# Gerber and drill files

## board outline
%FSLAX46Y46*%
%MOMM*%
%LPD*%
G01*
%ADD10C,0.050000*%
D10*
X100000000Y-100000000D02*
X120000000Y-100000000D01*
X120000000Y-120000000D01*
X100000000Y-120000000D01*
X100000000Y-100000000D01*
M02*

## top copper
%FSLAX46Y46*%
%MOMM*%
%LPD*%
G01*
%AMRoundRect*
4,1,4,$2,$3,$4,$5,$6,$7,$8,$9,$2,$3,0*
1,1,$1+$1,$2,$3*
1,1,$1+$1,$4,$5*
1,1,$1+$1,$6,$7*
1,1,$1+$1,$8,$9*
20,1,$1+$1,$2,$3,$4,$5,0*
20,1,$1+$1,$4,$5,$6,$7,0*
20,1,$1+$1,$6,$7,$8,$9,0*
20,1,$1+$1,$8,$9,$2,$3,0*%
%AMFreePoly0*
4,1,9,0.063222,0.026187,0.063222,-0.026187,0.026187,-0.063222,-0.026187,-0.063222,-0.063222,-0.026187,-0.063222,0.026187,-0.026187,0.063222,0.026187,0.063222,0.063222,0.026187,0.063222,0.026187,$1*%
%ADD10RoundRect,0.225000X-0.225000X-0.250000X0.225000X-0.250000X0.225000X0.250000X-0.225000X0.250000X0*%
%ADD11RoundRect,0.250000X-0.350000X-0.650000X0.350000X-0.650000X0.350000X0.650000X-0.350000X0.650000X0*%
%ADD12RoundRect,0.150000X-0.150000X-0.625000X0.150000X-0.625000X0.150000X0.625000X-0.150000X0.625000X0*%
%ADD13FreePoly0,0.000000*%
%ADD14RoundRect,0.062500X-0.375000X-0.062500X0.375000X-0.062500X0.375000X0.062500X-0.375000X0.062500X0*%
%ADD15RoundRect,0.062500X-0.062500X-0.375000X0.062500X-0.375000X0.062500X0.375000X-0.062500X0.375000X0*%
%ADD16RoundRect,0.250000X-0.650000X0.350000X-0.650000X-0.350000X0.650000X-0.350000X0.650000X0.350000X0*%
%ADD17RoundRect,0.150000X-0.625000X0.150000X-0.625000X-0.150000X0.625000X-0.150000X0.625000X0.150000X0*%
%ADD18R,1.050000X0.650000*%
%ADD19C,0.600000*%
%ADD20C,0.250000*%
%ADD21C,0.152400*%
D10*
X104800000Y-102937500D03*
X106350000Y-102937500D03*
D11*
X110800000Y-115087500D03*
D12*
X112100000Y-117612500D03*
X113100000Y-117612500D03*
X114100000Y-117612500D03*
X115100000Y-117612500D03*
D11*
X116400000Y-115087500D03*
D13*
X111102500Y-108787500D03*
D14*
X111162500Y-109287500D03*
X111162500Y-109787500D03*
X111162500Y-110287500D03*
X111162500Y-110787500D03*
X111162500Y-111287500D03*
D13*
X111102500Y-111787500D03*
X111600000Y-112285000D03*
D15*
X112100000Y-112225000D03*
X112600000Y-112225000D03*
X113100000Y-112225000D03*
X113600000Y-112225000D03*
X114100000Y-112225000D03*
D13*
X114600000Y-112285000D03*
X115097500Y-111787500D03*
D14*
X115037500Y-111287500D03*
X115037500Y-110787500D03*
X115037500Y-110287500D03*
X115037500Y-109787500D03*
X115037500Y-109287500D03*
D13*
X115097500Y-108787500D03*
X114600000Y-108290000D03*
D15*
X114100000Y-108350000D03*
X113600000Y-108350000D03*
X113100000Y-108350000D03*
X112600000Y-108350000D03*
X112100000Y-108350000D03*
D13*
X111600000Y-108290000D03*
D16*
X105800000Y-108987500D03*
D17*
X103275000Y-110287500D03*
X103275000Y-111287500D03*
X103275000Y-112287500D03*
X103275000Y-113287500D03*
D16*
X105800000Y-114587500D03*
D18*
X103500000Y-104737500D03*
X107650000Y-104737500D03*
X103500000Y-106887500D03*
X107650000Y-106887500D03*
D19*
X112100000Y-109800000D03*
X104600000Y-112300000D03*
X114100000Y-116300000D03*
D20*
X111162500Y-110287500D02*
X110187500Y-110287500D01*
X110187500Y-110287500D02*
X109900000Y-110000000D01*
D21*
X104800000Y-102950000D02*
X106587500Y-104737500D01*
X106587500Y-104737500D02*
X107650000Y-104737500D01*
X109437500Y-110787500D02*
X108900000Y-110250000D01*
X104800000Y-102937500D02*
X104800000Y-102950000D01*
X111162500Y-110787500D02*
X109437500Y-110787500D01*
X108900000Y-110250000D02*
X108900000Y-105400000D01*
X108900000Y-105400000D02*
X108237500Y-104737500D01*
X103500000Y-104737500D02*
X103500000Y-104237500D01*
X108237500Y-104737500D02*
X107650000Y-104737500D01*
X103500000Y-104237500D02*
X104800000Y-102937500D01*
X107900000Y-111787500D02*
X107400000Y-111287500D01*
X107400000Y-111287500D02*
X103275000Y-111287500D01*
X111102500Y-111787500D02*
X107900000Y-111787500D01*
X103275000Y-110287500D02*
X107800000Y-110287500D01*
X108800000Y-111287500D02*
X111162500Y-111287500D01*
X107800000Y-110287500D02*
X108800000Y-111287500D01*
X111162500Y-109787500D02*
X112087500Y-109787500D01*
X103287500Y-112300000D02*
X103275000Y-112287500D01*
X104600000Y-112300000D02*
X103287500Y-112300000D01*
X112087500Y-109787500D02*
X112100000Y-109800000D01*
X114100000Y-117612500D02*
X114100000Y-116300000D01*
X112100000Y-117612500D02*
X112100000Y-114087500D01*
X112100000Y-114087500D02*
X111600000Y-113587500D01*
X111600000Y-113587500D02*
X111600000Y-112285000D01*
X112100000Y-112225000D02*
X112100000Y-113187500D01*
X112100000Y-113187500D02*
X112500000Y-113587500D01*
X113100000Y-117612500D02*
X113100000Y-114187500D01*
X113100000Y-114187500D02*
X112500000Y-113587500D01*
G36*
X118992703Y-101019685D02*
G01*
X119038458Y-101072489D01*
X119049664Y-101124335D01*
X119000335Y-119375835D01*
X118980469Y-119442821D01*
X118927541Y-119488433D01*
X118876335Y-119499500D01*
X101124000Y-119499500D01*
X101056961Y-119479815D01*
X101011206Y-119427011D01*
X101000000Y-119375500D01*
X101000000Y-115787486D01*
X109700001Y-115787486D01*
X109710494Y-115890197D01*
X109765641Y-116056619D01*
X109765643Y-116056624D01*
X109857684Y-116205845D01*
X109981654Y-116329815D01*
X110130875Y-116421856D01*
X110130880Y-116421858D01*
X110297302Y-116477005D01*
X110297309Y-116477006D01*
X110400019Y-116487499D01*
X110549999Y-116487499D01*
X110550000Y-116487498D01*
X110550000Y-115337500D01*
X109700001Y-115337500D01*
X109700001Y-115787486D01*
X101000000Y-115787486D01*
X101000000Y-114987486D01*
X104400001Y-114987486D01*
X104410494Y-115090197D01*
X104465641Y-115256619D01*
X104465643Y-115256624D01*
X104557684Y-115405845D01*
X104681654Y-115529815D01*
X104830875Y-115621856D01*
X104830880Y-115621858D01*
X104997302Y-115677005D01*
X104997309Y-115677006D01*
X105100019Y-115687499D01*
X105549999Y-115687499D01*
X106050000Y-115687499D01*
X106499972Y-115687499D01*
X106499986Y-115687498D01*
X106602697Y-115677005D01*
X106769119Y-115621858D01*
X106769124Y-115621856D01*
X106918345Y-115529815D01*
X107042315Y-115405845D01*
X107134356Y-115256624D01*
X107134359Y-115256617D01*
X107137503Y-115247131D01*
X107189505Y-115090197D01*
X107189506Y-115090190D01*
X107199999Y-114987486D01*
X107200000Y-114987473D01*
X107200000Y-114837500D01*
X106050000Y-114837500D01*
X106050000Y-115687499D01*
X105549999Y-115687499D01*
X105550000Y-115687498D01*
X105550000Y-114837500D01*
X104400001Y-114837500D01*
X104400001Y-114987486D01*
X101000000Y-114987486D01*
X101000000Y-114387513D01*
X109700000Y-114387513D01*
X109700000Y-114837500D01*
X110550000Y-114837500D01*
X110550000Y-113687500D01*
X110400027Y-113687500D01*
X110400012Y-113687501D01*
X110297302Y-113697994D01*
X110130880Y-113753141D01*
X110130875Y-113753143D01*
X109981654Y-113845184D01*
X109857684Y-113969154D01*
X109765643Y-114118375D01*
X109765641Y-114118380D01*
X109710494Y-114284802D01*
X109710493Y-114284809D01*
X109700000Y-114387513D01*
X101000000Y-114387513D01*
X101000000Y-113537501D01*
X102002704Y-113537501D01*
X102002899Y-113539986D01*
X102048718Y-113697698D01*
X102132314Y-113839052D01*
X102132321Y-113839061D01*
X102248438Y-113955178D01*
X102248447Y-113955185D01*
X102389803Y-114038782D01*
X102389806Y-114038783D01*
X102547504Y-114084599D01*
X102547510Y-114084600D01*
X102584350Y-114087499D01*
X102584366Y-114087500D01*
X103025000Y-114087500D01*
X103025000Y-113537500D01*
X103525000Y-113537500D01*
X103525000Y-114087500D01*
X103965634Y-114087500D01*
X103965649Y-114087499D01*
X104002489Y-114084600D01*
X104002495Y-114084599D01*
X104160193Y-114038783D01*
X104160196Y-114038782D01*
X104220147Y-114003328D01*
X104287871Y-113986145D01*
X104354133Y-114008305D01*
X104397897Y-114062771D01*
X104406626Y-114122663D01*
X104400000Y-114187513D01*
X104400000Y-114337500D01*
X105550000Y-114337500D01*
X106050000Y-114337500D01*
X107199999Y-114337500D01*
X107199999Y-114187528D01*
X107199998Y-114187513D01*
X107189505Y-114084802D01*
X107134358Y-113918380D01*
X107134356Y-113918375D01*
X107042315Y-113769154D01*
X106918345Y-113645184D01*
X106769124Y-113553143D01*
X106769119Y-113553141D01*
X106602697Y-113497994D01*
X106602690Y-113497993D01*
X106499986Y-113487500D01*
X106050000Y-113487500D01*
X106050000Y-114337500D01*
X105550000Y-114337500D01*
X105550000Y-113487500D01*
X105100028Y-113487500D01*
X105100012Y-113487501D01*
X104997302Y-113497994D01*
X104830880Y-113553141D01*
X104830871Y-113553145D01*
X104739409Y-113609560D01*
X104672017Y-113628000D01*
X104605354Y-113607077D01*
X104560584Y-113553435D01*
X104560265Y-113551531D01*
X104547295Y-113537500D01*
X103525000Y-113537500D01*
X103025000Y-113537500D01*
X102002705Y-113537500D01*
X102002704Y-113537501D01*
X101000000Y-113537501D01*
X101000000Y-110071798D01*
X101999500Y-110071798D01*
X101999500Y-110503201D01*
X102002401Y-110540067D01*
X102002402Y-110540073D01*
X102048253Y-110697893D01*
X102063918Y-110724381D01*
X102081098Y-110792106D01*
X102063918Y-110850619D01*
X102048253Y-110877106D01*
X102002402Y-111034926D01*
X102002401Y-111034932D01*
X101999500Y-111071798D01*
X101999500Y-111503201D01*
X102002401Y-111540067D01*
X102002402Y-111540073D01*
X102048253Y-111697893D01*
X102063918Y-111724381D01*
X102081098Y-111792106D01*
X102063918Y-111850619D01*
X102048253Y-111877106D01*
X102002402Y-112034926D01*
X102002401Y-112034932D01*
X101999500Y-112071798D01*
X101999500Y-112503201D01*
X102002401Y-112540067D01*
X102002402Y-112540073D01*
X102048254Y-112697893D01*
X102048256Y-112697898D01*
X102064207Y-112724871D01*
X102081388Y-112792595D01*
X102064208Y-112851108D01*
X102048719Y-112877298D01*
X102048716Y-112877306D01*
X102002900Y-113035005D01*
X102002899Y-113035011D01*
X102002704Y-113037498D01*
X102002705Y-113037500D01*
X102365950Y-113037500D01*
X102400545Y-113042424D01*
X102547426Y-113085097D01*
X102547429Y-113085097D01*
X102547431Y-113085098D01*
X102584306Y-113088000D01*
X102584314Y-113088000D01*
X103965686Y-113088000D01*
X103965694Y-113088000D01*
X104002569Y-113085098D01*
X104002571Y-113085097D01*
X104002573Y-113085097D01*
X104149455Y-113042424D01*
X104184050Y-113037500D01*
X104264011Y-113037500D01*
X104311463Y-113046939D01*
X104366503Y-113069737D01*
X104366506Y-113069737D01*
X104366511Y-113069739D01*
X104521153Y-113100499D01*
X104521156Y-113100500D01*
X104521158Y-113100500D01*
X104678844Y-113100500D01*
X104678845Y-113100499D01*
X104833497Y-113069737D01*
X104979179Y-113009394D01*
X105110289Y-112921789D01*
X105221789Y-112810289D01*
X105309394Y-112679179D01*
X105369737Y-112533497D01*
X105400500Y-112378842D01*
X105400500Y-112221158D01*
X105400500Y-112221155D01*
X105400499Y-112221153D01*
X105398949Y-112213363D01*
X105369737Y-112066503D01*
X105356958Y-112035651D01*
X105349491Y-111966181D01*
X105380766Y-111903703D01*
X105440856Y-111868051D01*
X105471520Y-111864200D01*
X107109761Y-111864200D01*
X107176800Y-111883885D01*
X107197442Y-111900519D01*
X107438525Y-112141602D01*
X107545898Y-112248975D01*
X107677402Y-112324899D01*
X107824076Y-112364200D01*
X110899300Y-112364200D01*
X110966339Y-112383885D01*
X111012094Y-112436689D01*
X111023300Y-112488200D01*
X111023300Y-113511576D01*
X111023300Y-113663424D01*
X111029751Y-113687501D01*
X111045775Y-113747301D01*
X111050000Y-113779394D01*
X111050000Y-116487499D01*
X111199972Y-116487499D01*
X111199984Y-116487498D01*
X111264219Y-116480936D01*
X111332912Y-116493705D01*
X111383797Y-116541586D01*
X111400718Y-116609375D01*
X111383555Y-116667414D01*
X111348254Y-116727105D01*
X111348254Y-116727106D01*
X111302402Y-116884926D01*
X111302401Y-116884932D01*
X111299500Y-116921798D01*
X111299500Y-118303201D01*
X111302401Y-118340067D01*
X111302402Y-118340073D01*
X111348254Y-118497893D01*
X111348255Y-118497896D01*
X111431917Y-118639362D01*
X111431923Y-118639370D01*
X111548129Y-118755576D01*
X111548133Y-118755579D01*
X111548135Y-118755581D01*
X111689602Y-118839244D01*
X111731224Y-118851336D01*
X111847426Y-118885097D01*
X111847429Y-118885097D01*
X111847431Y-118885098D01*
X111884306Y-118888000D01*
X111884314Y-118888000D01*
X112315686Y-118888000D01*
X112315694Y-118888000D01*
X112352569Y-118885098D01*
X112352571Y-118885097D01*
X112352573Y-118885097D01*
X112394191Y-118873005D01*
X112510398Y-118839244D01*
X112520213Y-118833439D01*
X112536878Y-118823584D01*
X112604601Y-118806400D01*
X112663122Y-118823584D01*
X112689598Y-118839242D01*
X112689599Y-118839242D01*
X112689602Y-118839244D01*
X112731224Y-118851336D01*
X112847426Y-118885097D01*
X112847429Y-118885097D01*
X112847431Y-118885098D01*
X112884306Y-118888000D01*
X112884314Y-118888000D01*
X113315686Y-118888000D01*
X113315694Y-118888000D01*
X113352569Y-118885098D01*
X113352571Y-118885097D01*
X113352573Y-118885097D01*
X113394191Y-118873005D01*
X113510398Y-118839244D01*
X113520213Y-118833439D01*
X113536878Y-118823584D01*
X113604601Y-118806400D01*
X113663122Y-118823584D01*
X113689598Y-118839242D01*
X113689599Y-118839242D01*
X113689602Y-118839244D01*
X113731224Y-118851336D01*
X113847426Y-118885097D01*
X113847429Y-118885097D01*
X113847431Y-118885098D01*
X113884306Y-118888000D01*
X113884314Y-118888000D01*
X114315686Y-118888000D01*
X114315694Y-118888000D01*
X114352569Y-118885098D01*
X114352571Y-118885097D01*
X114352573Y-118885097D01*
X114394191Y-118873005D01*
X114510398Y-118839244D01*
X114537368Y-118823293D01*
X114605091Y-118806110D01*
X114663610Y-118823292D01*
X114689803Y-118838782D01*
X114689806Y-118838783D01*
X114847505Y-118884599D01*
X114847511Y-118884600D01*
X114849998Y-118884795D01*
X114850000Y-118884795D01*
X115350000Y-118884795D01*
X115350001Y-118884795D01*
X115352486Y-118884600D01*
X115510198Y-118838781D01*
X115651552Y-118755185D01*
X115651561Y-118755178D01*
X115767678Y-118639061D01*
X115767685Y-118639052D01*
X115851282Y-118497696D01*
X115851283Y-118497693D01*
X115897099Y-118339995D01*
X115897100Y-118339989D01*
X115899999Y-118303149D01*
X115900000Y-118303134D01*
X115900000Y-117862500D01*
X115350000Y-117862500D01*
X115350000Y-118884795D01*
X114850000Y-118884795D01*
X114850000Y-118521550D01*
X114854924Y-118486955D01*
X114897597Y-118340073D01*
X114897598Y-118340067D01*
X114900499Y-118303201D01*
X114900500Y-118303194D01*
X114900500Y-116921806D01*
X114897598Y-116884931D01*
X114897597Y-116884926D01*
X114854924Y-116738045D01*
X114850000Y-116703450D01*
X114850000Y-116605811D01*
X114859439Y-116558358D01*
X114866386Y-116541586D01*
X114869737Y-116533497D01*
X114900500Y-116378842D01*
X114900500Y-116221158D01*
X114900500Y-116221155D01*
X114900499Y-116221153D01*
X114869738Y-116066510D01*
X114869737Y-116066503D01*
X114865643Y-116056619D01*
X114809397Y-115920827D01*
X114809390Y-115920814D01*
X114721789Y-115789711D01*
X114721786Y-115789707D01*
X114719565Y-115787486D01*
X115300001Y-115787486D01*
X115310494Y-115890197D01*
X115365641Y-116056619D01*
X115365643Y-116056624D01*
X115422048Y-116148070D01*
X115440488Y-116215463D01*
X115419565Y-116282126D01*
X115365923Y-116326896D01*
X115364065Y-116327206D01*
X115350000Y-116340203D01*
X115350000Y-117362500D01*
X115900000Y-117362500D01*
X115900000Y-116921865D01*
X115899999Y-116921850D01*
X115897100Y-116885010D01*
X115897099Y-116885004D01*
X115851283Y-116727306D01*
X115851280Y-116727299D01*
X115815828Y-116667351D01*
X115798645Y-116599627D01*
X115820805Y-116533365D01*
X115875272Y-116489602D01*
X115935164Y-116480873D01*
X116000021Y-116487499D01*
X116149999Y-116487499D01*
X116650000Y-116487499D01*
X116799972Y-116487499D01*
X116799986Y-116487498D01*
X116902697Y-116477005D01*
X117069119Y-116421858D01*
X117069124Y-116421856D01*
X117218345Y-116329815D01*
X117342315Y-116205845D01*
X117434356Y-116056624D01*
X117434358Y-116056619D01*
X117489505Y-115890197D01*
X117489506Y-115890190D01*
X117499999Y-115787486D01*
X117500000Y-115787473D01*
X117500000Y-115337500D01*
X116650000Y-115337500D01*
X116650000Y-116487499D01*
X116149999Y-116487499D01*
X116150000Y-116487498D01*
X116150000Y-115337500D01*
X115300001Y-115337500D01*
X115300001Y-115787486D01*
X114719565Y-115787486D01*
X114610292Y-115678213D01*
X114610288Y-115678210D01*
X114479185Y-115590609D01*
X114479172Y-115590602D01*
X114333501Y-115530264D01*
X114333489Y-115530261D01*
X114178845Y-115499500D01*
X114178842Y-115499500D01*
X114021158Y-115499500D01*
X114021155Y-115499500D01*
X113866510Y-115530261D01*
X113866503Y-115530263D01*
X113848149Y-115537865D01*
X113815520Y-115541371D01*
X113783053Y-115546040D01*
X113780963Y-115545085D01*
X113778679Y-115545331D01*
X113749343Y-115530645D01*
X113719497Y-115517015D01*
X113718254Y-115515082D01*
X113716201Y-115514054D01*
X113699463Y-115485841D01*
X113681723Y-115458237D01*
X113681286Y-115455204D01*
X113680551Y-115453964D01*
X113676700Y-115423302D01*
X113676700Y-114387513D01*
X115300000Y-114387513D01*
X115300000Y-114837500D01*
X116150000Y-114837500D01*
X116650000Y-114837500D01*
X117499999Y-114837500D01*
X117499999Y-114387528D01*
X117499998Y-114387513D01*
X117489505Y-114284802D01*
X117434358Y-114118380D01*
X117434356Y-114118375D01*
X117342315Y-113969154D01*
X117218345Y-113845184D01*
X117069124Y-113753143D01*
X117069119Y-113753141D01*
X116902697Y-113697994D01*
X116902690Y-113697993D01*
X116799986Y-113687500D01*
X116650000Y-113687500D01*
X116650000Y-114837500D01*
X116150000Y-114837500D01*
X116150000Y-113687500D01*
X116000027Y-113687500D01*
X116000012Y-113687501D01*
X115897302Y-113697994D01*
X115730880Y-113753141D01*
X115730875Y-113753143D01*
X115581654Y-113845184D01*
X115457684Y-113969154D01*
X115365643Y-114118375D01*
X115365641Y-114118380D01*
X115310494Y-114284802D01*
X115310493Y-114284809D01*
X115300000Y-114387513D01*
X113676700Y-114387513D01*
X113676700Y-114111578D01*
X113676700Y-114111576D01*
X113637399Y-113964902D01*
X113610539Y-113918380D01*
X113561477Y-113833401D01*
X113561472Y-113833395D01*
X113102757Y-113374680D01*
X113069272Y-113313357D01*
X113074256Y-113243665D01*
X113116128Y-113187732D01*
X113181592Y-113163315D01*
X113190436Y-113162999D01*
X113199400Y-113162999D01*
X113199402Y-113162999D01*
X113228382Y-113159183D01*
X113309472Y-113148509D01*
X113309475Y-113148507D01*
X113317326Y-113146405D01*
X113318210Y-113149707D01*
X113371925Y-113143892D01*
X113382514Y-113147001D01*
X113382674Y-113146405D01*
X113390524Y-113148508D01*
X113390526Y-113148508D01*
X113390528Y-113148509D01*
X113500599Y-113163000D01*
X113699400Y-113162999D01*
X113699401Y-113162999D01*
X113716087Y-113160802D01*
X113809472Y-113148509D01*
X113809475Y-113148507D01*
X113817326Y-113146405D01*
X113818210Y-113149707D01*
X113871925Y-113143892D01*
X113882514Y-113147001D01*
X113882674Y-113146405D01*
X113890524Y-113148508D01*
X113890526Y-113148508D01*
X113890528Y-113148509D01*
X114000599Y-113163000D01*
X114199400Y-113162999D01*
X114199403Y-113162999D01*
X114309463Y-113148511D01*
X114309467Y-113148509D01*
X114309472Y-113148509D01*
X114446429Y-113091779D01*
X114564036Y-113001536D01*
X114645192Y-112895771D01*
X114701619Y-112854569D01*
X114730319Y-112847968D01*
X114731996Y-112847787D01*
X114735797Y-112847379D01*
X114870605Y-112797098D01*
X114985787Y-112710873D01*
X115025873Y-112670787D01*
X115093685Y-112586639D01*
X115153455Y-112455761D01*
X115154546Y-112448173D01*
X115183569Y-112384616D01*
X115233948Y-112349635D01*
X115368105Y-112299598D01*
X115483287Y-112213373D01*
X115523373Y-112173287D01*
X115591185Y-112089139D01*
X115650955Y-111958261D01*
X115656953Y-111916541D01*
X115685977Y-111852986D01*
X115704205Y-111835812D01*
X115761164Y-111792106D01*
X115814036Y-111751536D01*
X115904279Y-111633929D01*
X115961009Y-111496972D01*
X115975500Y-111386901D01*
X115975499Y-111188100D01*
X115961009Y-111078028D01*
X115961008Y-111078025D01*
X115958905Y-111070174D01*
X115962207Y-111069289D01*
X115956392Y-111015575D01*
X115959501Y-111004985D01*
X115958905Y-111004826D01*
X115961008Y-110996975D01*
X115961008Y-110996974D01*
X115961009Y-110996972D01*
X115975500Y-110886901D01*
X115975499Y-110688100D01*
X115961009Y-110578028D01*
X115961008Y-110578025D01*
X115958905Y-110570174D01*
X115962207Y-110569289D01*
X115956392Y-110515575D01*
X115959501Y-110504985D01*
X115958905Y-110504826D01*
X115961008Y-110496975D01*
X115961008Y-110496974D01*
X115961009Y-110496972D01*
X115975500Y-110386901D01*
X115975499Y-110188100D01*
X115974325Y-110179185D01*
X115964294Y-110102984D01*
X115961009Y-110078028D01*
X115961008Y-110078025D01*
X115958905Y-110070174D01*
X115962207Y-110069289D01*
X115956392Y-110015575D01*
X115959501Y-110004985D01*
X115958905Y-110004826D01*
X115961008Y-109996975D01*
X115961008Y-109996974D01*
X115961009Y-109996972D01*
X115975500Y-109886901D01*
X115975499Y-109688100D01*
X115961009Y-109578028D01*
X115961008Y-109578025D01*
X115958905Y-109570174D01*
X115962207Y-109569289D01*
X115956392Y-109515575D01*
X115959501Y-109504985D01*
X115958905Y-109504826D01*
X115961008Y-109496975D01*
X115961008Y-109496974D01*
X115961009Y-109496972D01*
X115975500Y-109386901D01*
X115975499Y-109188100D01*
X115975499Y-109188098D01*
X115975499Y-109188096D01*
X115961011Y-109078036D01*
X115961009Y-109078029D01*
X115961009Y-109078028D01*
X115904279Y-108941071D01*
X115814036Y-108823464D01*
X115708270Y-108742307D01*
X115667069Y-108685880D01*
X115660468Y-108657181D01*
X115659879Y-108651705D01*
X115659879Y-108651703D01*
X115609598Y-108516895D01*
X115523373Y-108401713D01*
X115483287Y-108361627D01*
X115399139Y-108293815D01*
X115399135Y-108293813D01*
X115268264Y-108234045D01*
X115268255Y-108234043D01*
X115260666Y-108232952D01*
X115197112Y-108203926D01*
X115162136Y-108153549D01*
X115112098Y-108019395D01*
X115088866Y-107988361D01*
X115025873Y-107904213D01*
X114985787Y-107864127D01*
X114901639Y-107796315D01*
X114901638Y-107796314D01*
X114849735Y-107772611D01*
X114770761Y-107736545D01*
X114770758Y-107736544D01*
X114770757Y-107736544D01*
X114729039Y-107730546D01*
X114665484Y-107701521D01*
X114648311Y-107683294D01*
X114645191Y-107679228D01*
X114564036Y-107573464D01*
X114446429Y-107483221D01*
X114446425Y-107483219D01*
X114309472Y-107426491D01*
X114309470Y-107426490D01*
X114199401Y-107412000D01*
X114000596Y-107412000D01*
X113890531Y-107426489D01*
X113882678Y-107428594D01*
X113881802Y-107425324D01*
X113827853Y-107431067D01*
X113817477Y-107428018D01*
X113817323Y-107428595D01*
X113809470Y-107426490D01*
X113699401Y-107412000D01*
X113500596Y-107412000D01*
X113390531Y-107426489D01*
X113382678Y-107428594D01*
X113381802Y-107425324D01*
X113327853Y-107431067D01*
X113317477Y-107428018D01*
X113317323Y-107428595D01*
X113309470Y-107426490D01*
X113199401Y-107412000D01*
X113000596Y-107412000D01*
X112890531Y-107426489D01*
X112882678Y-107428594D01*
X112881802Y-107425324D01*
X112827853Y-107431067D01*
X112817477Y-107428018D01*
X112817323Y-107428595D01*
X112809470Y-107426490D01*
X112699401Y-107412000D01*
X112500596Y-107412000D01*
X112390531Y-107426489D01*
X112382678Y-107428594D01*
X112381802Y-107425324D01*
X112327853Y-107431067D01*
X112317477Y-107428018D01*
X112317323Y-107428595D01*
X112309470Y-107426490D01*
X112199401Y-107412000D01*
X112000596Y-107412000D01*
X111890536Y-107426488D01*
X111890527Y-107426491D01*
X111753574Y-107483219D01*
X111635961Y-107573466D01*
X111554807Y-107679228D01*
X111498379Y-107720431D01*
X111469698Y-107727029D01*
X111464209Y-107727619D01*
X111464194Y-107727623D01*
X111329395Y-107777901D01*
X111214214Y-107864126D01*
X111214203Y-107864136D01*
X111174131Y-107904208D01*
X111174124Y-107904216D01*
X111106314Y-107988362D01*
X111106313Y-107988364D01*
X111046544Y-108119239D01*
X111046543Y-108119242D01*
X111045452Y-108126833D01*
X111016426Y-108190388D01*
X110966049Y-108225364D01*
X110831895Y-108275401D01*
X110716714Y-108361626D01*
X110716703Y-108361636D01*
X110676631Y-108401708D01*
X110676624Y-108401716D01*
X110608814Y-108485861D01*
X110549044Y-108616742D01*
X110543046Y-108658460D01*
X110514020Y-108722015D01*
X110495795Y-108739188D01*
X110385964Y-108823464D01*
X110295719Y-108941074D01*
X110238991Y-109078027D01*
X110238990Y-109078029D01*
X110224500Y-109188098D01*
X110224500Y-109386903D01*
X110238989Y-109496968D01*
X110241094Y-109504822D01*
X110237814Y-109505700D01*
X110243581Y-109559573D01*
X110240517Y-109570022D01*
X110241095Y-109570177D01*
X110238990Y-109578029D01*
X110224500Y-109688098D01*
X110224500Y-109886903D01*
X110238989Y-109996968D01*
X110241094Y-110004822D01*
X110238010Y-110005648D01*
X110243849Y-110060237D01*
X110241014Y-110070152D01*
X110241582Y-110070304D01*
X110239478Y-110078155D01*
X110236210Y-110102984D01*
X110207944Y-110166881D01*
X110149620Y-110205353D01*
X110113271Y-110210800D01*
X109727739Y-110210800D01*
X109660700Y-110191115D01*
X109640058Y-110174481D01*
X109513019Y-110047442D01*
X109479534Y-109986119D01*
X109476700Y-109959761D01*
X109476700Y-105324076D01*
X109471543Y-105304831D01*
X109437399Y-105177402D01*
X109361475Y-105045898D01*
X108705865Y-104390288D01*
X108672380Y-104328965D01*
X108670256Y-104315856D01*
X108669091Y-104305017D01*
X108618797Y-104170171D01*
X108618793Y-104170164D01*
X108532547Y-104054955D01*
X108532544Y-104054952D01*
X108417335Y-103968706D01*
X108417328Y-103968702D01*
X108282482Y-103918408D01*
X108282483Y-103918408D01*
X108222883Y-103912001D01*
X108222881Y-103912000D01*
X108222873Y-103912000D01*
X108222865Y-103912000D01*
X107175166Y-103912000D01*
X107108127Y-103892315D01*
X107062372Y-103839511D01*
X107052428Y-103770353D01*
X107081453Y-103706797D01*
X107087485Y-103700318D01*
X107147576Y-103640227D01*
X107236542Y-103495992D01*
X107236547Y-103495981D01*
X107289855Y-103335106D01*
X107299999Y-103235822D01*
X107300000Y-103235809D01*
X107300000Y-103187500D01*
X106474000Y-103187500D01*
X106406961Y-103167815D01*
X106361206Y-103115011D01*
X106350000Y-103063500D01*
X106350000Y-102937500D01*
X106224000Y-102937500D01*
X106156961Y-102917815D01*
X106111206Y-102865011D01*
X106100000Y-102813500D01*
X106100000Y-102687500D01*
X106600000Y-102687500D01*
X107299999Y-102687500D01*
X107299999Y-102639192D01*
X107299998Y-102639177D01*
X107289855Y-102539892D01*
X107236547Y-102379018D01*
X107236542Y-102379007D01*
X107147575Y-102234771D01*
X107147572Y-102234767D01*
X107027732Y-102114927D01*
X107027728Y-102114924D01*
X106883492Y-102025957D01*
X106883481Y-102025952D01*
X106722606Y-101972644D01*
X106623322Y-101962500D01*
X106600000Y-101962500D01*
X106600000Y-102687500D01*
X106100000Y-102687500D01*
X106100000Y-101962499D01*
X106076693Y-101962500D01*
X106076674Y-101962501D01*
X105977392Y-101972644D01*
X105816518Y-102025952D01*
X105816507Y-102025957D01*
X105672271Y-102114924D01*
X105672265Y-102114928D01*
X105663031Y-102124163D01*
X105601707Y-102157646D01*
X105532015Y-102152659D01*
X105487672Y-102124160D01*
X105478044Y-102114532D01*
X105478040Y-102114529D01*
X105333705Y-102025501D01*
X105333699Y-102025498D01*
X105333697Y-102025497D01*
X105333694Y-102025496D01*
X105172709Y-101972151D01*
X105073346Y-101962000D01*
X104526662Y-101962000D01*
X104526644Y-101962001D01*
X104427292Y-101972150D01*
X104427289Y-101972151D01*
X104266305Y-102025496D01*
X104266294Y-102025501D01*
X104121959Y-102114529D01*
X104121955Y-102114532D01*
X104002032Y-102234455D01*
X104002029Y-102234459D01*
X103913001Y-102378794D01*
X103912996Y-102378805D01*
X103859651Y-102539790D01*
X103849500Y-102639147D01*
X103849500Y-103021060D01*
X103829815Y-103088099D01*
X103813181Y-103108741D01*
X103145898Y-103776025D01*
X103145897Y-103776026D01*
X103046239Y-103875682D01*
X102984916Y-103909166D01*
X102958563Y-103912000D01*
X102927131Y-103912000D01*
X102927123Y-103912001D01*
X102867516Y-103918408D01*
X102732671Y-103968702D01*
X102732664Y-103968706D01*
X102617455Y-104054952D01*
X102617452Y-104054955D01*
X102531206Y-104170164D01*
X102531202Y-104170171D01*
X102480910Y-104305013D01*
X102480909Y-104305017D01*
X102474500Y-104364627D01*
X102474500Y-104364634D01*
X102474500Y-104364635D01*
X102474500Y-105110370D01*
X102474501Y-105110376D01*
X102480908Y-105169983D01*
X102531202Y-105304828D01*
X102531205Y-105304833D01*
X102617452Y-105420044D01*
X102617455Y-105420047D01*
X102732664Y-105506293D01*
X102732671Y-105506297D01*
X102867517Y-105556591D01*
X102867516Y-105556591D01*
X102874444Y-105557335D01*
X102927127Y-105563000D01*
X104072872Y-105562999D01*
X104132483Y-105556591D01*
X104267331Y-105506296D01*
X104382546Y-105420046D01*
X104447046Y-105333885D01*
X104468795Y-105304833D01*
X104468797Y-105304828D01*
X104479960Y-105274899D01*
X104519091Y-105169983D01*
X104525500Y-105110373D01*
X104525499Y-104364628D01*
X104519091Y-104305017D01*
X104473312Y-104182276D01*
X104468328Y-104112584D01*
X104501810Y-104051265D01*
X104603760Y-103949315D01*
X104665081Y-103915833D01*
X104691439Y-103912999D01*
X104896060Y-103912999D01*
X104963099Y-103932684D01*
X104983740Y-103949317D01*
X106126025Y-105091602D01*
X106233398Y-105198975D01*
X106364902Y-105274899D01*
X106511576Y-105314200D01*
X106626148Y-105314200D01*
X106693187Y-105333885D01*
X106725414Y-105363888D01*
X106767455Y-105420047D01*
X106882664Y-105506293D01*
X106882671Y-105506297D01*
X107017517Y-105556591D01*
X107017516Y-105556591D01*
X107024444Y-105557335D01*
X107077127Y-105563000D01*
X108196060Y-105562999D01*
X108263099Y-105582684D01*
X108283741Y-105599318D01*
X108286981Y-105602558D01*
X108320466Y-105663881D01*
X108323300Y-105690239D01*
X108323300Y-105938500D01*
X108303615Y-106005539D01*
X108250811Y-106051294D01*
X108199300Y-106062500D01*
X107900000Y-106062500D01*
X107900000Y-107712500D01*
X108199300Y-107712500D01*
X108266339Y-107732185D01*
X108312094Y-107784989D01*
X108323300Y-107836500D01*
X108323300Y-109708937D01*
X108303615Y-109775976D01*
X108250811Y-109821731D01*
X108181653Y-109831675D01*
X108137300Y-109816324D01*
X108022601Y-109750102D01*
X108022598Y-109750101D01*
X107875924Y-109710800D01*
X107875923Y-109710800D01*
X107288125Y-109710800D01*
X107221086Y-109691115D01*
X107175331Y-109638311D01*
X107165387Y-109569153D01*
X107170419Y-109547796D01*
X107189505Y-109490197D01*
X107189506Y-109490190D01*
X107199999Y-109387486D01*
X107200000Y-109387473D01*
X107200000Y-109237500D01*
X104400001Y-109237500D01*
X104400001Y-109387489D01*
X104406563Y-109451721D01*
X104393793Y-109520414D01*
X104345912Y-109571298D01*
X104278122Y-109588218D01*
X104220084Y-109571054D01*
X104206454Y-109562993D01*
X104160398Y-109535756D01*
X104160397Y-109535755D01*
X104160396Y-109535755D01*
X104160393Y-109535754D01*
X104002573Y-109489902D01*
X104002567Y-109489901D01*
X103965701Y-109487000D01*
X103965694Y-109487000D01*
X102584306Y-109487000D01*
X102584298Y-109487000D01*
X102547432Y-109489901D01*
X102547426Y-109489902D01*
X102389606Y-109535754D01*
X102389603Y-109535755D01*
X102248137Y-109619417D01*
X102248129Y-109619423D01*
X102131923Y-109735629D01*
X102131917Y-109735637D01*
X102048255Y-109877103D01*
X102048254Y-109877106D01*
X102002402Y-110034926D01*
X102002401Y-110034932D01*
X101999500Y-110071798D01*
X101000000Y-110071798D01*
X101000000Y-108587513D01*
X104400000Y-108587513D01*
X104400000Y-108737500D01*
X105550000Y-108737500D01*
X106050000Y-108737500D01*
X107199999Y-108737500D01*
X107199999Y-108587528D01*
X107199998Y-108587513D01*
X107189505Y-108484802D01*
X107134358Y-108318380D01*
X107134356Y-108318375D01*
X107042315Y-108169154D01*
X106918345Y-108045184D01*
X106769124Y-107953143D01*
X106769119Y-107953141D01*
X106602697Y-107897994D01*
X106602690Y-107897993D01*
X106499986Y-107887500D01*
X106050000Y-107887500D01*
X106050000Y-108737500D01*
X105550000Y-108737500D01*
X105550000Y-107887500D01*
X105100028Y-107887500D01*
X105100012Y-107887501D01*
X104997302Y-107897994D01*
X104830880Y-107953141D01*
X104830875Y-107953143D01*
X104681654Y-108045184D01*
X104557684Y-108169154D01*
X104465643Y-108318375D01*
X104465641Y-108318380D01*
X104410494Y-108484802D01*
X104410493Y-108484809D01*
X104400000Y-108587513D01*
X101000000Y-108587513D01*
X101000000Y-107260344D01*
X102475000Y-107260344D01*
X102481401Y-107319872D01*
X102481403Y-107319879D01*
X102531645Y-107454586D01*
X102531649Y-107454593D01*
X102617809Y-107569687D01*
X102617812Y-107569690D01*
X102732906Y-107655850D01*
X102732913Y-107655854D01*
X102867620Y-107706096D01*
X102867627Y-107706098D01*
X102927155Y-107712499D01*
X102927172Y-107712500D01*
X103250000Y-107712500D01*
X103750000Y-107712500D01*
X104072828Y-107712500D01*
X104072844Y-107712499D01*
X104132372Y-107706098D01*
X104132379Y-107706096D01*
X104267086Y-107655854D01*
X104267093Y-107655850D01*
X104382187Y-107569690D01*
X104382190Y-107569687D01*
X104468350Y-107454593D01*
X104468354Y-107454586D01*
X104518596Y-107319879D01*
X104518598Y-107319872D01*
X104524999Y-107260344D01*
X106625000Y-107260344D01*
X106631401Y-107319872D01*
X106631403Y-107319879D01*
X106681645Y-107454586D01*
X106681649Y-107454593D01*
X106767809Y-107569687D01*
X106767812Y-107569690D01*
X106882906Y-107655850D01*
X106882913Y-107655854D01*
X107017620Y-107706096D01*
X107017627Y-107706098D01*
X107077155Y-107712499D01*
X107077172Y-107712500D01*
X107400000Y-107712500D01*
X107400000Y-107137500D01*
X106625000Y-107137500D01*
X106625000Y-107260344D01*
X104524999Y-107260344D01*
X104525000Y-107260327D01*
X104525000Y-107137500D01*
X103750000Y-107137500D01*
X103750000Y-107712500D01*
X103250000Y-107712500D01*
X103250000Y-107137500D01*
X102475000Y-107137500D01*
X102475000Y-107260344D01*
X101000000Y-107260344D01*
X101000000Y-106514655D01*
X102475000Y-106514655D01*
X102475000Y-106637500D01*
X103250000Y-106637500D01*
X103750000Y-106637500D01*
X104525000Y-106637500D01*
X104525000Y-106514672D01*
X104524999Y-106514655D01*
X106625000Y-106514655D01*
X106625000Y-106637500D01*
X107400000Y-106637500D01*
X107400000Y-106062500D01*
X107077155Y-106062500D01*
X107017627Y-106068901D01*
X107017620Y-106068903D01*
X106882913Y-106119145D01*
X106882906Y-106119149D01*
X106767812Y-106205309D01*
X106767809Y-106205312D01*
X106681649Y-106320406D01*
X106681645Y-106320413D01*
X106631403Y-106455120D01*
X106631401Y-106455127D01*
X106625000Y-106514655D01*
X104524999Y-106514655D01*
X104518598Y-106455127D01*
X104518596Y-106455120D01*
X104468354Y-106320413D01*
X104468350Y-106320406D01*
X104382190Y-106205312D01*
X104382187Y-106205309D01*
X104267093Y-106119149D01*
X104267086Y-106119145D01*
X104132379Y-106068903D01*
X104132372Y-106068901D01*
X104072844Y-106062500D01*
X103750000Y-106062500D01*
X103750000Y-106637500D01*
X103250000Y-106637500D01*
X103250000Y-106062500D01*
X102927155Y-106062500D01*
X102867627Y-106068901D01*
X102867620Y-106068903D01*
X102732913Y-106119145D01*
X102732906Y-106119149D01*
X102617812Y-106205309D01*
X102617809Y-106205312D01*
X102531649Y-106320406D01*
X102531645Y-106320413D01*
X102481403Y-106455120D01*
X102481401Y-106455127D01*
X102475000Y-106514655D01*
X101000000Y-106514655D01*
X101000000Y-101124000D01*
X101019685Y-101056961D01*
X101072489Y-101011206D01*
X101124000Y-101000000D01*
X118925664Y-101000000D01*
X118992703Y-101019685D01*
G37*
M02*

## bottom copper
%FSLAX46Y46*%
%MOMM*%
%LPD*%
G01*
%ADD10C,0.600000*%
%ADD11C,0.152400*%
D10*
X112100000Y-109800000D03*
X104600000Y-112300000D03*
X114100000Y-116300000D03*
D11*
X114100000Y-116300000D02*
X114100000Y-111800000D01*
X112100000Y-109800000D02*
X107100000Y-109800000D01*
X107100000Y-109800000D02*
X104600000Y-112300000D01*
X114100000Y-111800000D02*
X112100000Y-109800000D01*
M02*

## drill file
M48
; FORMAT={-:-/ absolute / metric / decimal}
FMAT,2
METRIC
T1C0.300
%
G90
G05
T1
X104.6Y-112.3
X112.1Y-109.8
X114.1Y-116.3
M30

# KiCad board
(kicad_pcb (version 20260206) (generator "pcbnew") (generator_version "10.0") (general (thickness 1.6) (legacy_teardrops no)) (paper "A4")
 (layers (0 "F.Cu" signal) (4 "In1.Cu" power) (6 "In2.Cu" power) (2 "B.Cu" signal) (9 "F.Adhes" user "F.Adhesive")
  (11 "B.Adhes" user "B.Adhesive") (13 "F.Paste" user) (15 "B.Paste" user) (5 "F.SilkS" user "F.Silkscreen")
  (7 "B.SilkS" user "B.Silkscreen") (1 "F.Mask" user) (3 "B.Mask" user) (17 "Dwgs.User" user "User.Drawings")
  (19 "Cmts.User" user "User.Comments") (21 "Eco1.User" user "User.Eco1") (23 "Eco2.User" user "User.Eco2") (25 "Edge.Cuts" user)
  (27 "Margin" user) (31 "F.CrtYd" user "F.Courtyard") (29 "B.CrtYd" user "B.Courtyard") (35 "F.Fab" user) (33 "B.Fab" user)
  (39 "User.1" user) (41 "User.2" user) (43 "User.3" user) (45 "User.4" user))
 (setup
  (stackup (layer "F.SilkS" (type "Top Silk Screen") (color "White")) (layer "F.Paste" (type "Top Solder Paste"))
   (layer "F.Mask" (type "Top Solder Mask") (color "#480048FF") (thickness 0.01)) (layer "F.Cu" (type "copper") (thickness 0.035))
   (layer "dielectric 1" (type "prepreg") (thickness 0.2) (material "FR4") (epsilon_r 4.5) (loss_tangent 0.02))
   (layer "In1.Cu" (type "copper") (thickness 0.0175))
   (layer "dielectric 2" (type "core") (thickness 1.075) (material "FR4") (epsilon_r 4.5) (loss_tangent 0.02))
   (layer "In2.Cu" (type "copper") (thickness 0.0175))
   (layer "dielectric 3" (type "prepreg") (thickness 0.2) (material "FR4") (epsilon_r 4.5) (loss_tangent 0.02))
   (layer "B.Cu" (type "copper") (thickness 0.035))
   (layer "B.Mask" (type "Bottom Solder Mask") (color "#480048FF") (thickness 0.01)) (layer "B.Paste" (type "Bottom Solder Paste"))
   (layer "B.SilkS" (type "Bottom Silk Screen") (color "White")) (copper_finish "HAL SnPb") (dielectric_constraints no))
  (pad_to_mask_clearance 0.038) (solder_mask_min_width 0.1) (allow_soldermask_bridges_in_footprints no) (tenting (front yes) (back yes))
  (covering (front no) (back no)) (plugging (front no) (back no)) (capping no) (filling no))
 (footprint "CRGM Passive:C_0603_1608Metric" (layer "F.Cu") (at 105.575 102.9375)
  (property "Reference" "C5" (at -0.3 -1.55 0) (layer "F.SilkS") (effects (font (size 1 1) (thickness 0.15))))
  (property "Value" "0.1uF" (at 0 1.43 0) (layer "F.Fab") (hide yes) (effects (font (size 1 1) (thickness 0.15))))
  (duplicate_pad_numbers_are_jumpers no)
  (pad "1" smd roundrect (at -0.775 0) (size 0.9 0.95) (layers "F.Cu" "F.Mask" "F.Paste") (roundrect_rratio 0.25) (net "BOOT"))
  (pad "2" smd roundrect (at 0.775 0) (size 0.9 0.95) (layers "F.Cu" "F.Mask" "F.Paste") (roundrect_rratio 0.25) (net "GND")))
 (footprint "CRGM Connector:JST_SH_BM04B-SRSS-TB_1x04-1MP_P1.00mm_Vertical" (layer "F.Cu") (at 113.6 116.2875)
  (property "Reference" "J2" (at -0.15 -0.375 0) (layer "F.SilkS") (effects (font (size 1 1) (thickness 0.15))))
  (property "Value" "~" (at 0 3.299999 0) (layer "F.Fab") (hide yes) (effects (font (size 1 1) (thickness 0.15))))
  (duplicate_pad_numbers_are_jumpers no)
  (pad "0" smd roundrect (at -2.8 -1.2) (size 1.2 1.8) (layers "F.Cu" "F.Mask" "F.Paste") (roundrect_rratio 0.208333) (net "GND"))
  (pad "1" smd roundrect (at -1.5 1.325) (size 0.6 1.55) (layers "F.Cu" "F.Mask" "F.Paste") (roundrect_rratio 0.25) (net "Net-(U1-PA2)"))
  (pad "2" smd roundrect (at -0.5 1.325) (size 0.6 1.55) (layers "F.Cu" "F.Mask" "F.Paste") (roundrect_rratio 0.25) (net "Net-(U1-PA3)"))
  (pad "3" smd roundrect (at 0.5 1.325) (size 0.6 1.55) (layers "F.Cu" "F.Mask" "F.Paste") (roundrect_rratio 0.25) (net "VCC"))
  (pad "4" smd roundrect (at 1.5 1.325) (size 0.6 1.55) (layers "F.Cu" "F.Mask" "F.Paste") (roundrect_rratio 0.25) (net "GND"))
  (pad "5" smd roundrect (at 2.8 -1.2) (size 1.2 1.8) (layers "F.Cu" "F.Mask" "F.Paste") (roundrect_rratio 0.208333) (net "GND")))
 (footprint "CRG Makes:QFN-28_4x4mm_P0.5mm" (layer "F.Cu") (at 113.1 110.2875)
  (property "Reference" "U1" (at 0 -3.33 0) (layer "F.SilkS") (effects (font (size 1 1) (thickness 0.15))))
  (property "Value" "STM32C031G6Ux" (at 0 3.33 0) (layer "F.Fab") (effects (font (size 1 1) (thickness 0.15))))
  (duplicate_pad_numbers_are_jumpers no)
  (pad "1" smd custom (at -1.9975 -1.5) (size 0.136863 0.136863) (layers "F.Cu" "F.Mask" "F.Paste")
   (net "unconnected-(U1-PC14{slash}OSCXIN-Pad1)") (options (clearance outline) (anchor circle)) (primitives))
  (pad "2" smd roundrect (at -1.9375 -1) (size 0.875 0.25) (layers "F.Cu" "F.Mask" "F.Paste") (roundrect_rratio 0.25)
   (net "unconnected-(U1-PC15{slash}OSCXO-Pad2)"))
  (pad "3" smd roundrect (at -1.9375 -0.5) (size 0.875 0.25) (layers "F.Cu" "F.Mask" "F.Paste") (roundrect_rratio 0.25) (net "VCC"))
  (pad "4" smd roundrect (at -1.9375 0) (size 0.875 0.25) (layers "F.Cu" "F.Mask" "F.Paste") (roundrect_rratio 0.25) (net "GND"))
  (pad "5" smd roundrect (at -1.9375 0.5) (size 0.875 0.25) (layers "F.Cu" "F.Mask" "F.Paste") (roundrect_rratio 0.25) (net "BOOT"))
  (pad "6" smd roundrect (at -1.9375 1) (size 0.875 0.25) (layers "F.Cu" "F.Mask" "F.Paste") (roundrect_rratio 0.25) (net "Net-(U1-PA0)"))
  (pad "7" smd custom (at -1.9975 1.5) (size 0.136863 0.136863) (layers "F.Cu" "F.Mask" "F.Paste") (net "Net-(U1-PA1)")
   (options (clearance outline) (anchor circle)) (primitives))
  (pad "8" smd custom (at -1.5 1.9975) (size 0.136863 0.136863) (layers "F.Cu" "F.Mask" "F.Paste") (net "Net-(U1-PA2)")
   (options (clearance outline) (anchor circle)) (primitives))
  (pad "9" smd roundrect (at -1 1.9375) (size 0.25 0.875) (layers "F.Cu" "F.Mask" "F.Paste") (roundrect_rratio 0.25) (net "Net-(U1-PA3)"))
  (pad "10" smd roundrect (at -0.5 1.9375) (size 0.25 0.875) (layers "F.Cu" "F.Mask" "F.Paste") (roundrect_rratio 0.25)
   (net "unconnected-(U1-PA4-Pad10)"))
  (pad "11" smd roundrect (at 0 1.9375) (size 0.25 0.875) (layers "F.Cu" "F.Mask" "F.Paste") (roundrect_rratio 0.25)
   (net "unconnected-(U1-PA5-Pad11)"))
  (pad "12" smd roundrect (at 0.5 1.9375) (size 0.25 0.875) (layers "F.Cu" "F.Mask" "F.Paste") (roundrect_rratio 0.25)
   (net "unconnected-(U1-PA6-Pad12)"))
  (pad "13" smd roundrect (at 1 1.9375) (size 0.25 0.875) (layers "F.Cu" "F.Mask" "F.Paste") (roundrect_rratio 0.25)
   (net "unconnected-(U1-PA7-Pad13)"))
  (pad "14" smd custom (at 1.5 1.9975) (size 0.136863 0.136863) (layers "F.Cu" "F.Mask" "F.Paste") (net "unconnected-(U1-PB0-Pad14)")
   (options (clearance outline) (anchor circle)) (primitives))
  (pad "15" smd custom (at 1.9975 1.5) (size 0.136863 0.136863) (layers "F.Cu" "F.Mask" "F.Paste") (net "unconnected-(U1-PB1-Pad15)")
   (options (clearance outline) (anchor circle)) (primitives))
  (pad "16" smd roundrect (at 1.9375 1) (size 0.875 0.25) (layers "F.Cu" "F.Mask" "F.Paste") (roundrect_rratio 0.25)
   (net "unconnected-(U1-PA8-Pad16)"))
  (pad "17" smd roundrect (at 1.9375 0.5) (size 0.875 0.25) (layers "F.Cu" "F.Mask" "F.Paste") (roundrect_rratio 0.25)
   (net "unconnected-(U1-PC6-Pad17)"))
  (pad "18" smd roundrect (at 1.9375 0) (size 0.875 0.25) (layers "F.Cu" "F.Mask" "F.Paste") (roundrect_rratio 0.25)
   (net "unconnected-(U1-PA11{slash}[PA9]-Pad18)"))
  (pad "19" smd roundrect (at 1.9375 -0.5) (size 0.875 0.25) (layers "F.Cu" "F.Mask" "F.Paste") (roundrect_rratio 0.25)
   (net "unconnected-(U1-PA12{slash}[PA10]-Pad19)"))
  (pad "20" smd roundrect (at 1.9375 -1) (size 0.875 0.25) (layers "F.Cu" "F.Mask" "F.Paste") (roundrect_rratio 0.25)
   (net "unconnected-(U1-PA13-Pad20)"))
  (pad "21" smd custom (at 1.9975 -1.5) (size 0.136863 0.136863) (layers "F.Cu" "F.Mask" "F.Paste")
   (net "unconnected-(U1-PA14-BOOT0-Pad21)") (options (clearance outline) (anchor circle)) (primitives))
  (pad "22" smd custom (at 1.5 -1.9975) (size 0.136863 0.136863) (layers "F.Cu" "F.Mask" "F.Paste") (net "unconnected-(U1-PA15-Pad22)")
   (options (clearance outline) (anchor circle)) (primitives))
  (pad "23" smd roundrect (at 1 -1.9375) (size 0.25 0.875) (layers "F.Cu" "F.Mask" "F.Paste") (roundrect_rratio 0.25)
   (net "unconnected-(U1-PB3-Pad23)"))
  (pad "24" smd roundrect (at 0.5 -1.9375) (size 0.25 0.875) (layers "F.Cu" "F.Mask" "F.Paste") (roundrect_rratio 0.25)
   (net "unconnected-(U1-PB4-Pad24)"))
  (pad "25" smd roundrect (at 0 -1.9375) (size 0.25 0.875) (layers "F.Cu" "F.Mask" "F.Paste") (roundrect_rratio 0.25)
   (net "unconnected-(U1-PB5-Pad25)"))
  (pad "26" smd roundrect (at -0.5 -1.9375) (size 0.25 0.875) (layers "F.Cu" "F.Mask" "F.Paste") (roundrect_rratio 0.25)
   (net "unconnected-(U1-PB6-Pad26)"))
  (pad "27" smd roundrect (at -1 -1.9375) (size 0.25 0.875) (layers "F.Cu" "F.Mask" "F.Paste") (roundrect_rratio 0.25)
   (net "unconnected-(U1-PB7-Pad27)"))
  (pad "28" smd custom (at -1.5 -1.9975) (size 0.136863 0.136863) (layers "F.Cu" "F.Mask" "F.Paste") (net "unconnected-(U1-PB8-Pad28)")
   (options (clearance outline) (anchor circle)) (primitives)))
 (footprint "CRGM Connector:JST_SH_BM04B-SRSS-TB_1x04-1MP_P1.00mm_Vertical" (layer "F.Cu") (at 104.6 111.7875 -90)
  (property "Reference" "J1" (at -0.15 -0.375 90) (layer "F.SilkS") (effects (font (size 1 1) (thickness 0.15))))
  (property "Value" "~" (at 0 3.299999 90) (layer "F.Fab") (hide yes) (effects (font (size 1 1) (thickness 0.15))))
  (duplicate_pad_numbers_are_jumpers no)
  (pad "0" smd roundrect (at -2.8 -1.2 270) (size 1.2 1.8) (layers "F.Cu" "F.Mask" "F.Paste") (roundrect_rratio 0.208333) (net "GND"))
  (pad "1" smd roundrect (at -1.5 1.325 270) (size 0.6 1.55) (layers "F.Cu" "F.Mask" "F.Paste") (roundrect_rratio 0.25) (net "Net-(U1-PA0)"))
  (pad "2" smd roundrect (at -0.5 1.325 270) (size 0.6 1.55) (layers "F.Cu" "F.Mask" "F.Paste") (roundrect_rratio 0.25) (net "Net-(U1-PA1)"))
  (pad "3" smd roundrect (at 0.5 1.325 270) (size 0.6 1.55) (layers "F.Cu" "F.Mask" "F.Paste") (roundrect_rratio 0.25) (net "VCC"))
  (pad "4" smd roundrect (at 1.5 1.325 270) (size 0.6 1.55) (layers "F.Cu" "F.Mask" "F.Paste") (roundrect_rratio 0.25) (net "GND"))
  (pad "5" smd roundrect (at 2.8 -1.2 270) (size 1.2 1.8) (layers "F.Cu" "F.Mask" "F.Paste") (roundrect_rratio 0.208333) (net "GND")))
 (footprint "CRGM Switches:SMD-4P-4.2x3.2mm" (layer "F.Cu") (at 105.575 105.8125)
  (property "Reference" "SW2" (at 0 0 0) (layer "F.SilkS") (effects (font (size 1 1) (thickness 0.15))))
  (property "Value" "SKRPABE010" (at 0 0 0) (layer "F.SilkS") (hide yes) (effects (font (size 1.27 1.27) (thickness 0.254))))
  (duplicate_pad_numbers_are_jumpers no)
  (pad "1" smd rect (at -2.075 -1.075 90) (size 0.65 1.05) (layers "F.Cu" "F.Mask" "F.Paste") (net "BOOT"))
  (pad "2" smd rect (at 2.075 -1.075 90) (size 0.65 1.05) (layers "F.Cu" "F.Mask" "F.Paste") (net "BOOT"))
  (pad "3" smd rect (at -2.075 1.075 90) (size 0.65 1.05) (layers "F.Cu" "F.Mask" "F.Paste") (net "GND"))
  (pad "4" smd rect (at 2.075 1.075 90) (size 0.65 1.05) (layers "F.Cu" "F.Mask" "F.Paste") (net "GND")))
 (gr_rect (start 100 100) (end 120 120) (stroke (width 0.05) (type default)) (fill no) (layer "Edge.Cuts"))
 (segment (start 111.1625 110.2875) (end 110.1875 110.2875) (width 0.25) (layer "F.Cu") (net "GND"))
 (segment (start 110.1875 110.2875) (end 109.9 110) (width 0.25) (layer "F.Cu") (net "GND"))
 (segment (start 104.8 102.95) (end 106.5875 104.7375) (width 0.1524) (layer "F.Cu") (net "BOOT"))
 (segment (start 106.5875 104.7375) (end 107.65 104.7375) (width 0.1524) (layer "F.Cu") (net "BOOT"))
 (segment (start 109.4375 110.7875) (end 108.9 110.25) (width 0.1524) (layer "F.Cu") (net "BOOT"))
 (segment (start 104.8 102.9375) (end 104.8 102.95) (width 0.1524) (layer "F.Cu") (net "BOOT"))
 (segment (start 111.1625 110.7875) (end 109.4375 110.7875) (width 0.1524) (layer "F.Cu") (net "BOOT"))
 (segment (start 108.9 110.25) (end 108.9 105.4) (width 0.1524) (layer "F.Cu") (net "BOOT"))
 (segment (start 108.9 105.4) (end 108.2375 104.7375) (width 0.1524) (layer "F.Cu") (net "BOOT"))
 (segment (start 103.5 104.7375) (end 103.5 104.2375) (width 0.1524) (layer "F.Cu") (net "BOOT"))
 (segment (start 108.2375 104.7375) (end 107.65 104.7375) (width 0.1524) (layer "F.Cu") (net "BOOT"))
 (segment (start 103.5 104.2375) (end 104.8 102.9375) (width 0.1524) (layer "F.Cu") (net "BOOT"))
 (segment (start 107.9 111.7875) (end 107.4 111.2875) (width 0.1524) (layer "F.Cu") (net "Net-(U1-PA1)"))
 (segment (start 107.4 111.2875) (end 103.275 111.2875) (width 0.1524) (layer "F.Cu") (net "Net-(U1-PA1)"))
 (segment (start 111.1025 111.7875) (end 107.9 111.7875) (width 0.1524) (layer "F.Cu") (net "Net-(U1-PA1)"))
 (segment (start 103.275 110.2875) (end 107.8 110.2875) (width 0.1524) (layer "F.Cu") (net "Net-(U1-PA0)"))
 (segment (start 108.8 111.2875) (end 111.1625 111.2875) (width 0.1524) (layer "F.Cu") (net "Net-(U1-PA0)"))
 (segment (start 107.8 110.2875) (end 108.8 111.2875) (width 0.1524) (layer "F.Cu") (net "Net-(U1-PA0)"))
 (segment (start 111.1625 109.7875) (end 112.0875 109.7875) (width 0.1524) (layer "F.Cu") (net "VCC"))
 (segment (start 103.2875 112.3) (end 103.275 112.2875) (width 0.1524) (layer "F.Cu") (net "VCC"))
 (segment (start 104.6 112.3) (end 103.2875 112.3) (width 0.1524) (layer "F.Cu") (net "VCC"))
 (segment (start 112.0875 109.7875) (end 112.1 109.8) (width 0.1524) (layer "F.Cu") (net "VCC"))
 (segment (start 114.1 117.6125) (end 114.1 116.3) (width 0.1524) (layer "F.Cu") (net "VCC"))
 (via (at 112.1 109.8) (size 0.6) (drill 0.3) (layers "F.Cu" "B.Cu") (capping no) (covering (front no) (back no))
  (plugging (front no) (back no)) (filling no) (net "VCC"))
 (via (at 104.6 112.3) (size 0.6) (drill 0.3) (layers "F.Cu" "B.Cu") (capping no) (covering (front no) (back no))
  (plugging (front no) (back no)) (filling no) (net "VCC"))
 (via (at 114.1 116.3) (size 0.6) (drill 0.3) (layers "F.Cu" "B.Cu") (capping no) (covering (front no) (back no))
  (plugging (front no) (back no)) (filling no) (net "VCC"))
 (segment (start 114.1 116.3) (end 114.1 111.8) (width 0.1524) (layer "B.Cu") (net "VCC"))
 (segment (start 112.1 109.8) (end 107.1 109.8) (width 0.1524) (layer "B.Cu") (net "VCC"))
 (segment (start 107.1 109.8) (end 104.6 112.3) (width 0.1524) (layer "B.Cu") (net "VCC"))
 (segment (start 114.1 111.8) (end 112.1 109.8) (width 0.1524) (layer "B.Cu") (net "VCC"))
 (segment (start 112.1 117.6125) (end 112.1 114.0875) (width 0.1524) (layer "F.Cu") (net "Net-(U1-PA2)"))
 (segment (start 112.1 114.0875) (end 111.6 113.5875) (width 0.1524) (layer "F.Cu") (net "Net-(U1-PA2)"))
 (segment (start 111.6 113.5875) (end 111.6 112.285) (width 0.1524) (layer "F.Cu") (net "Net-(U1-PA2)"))
 (segment (start 112.1 112.225) (end 112.1 113.1875) (width 0.1524) (layer "F.Cu") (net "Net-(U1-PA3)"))
 (segment (start 112.1 113.1875) (end 112.5 113.5875) (width 0.1524) (layer "F.Cu") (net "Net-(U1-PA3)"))
 (segment (start 113.1 117.6125) (end 113.1 114.1875) (width 0.1524) (layer "F.Cu") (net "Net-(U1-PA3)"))
 (segment (start 113.1 114.1875) (end 112.5 113.5875) (width 0.1524) (layer "F.Cu") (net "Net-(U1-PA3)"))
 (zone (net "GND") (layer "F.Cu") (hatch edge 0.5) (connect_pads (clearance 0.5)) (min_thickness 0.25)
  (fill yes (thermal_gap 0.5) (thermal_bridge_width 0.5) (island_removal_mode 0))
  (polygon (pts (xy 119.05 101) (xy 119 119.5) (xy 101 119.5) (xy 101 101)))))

